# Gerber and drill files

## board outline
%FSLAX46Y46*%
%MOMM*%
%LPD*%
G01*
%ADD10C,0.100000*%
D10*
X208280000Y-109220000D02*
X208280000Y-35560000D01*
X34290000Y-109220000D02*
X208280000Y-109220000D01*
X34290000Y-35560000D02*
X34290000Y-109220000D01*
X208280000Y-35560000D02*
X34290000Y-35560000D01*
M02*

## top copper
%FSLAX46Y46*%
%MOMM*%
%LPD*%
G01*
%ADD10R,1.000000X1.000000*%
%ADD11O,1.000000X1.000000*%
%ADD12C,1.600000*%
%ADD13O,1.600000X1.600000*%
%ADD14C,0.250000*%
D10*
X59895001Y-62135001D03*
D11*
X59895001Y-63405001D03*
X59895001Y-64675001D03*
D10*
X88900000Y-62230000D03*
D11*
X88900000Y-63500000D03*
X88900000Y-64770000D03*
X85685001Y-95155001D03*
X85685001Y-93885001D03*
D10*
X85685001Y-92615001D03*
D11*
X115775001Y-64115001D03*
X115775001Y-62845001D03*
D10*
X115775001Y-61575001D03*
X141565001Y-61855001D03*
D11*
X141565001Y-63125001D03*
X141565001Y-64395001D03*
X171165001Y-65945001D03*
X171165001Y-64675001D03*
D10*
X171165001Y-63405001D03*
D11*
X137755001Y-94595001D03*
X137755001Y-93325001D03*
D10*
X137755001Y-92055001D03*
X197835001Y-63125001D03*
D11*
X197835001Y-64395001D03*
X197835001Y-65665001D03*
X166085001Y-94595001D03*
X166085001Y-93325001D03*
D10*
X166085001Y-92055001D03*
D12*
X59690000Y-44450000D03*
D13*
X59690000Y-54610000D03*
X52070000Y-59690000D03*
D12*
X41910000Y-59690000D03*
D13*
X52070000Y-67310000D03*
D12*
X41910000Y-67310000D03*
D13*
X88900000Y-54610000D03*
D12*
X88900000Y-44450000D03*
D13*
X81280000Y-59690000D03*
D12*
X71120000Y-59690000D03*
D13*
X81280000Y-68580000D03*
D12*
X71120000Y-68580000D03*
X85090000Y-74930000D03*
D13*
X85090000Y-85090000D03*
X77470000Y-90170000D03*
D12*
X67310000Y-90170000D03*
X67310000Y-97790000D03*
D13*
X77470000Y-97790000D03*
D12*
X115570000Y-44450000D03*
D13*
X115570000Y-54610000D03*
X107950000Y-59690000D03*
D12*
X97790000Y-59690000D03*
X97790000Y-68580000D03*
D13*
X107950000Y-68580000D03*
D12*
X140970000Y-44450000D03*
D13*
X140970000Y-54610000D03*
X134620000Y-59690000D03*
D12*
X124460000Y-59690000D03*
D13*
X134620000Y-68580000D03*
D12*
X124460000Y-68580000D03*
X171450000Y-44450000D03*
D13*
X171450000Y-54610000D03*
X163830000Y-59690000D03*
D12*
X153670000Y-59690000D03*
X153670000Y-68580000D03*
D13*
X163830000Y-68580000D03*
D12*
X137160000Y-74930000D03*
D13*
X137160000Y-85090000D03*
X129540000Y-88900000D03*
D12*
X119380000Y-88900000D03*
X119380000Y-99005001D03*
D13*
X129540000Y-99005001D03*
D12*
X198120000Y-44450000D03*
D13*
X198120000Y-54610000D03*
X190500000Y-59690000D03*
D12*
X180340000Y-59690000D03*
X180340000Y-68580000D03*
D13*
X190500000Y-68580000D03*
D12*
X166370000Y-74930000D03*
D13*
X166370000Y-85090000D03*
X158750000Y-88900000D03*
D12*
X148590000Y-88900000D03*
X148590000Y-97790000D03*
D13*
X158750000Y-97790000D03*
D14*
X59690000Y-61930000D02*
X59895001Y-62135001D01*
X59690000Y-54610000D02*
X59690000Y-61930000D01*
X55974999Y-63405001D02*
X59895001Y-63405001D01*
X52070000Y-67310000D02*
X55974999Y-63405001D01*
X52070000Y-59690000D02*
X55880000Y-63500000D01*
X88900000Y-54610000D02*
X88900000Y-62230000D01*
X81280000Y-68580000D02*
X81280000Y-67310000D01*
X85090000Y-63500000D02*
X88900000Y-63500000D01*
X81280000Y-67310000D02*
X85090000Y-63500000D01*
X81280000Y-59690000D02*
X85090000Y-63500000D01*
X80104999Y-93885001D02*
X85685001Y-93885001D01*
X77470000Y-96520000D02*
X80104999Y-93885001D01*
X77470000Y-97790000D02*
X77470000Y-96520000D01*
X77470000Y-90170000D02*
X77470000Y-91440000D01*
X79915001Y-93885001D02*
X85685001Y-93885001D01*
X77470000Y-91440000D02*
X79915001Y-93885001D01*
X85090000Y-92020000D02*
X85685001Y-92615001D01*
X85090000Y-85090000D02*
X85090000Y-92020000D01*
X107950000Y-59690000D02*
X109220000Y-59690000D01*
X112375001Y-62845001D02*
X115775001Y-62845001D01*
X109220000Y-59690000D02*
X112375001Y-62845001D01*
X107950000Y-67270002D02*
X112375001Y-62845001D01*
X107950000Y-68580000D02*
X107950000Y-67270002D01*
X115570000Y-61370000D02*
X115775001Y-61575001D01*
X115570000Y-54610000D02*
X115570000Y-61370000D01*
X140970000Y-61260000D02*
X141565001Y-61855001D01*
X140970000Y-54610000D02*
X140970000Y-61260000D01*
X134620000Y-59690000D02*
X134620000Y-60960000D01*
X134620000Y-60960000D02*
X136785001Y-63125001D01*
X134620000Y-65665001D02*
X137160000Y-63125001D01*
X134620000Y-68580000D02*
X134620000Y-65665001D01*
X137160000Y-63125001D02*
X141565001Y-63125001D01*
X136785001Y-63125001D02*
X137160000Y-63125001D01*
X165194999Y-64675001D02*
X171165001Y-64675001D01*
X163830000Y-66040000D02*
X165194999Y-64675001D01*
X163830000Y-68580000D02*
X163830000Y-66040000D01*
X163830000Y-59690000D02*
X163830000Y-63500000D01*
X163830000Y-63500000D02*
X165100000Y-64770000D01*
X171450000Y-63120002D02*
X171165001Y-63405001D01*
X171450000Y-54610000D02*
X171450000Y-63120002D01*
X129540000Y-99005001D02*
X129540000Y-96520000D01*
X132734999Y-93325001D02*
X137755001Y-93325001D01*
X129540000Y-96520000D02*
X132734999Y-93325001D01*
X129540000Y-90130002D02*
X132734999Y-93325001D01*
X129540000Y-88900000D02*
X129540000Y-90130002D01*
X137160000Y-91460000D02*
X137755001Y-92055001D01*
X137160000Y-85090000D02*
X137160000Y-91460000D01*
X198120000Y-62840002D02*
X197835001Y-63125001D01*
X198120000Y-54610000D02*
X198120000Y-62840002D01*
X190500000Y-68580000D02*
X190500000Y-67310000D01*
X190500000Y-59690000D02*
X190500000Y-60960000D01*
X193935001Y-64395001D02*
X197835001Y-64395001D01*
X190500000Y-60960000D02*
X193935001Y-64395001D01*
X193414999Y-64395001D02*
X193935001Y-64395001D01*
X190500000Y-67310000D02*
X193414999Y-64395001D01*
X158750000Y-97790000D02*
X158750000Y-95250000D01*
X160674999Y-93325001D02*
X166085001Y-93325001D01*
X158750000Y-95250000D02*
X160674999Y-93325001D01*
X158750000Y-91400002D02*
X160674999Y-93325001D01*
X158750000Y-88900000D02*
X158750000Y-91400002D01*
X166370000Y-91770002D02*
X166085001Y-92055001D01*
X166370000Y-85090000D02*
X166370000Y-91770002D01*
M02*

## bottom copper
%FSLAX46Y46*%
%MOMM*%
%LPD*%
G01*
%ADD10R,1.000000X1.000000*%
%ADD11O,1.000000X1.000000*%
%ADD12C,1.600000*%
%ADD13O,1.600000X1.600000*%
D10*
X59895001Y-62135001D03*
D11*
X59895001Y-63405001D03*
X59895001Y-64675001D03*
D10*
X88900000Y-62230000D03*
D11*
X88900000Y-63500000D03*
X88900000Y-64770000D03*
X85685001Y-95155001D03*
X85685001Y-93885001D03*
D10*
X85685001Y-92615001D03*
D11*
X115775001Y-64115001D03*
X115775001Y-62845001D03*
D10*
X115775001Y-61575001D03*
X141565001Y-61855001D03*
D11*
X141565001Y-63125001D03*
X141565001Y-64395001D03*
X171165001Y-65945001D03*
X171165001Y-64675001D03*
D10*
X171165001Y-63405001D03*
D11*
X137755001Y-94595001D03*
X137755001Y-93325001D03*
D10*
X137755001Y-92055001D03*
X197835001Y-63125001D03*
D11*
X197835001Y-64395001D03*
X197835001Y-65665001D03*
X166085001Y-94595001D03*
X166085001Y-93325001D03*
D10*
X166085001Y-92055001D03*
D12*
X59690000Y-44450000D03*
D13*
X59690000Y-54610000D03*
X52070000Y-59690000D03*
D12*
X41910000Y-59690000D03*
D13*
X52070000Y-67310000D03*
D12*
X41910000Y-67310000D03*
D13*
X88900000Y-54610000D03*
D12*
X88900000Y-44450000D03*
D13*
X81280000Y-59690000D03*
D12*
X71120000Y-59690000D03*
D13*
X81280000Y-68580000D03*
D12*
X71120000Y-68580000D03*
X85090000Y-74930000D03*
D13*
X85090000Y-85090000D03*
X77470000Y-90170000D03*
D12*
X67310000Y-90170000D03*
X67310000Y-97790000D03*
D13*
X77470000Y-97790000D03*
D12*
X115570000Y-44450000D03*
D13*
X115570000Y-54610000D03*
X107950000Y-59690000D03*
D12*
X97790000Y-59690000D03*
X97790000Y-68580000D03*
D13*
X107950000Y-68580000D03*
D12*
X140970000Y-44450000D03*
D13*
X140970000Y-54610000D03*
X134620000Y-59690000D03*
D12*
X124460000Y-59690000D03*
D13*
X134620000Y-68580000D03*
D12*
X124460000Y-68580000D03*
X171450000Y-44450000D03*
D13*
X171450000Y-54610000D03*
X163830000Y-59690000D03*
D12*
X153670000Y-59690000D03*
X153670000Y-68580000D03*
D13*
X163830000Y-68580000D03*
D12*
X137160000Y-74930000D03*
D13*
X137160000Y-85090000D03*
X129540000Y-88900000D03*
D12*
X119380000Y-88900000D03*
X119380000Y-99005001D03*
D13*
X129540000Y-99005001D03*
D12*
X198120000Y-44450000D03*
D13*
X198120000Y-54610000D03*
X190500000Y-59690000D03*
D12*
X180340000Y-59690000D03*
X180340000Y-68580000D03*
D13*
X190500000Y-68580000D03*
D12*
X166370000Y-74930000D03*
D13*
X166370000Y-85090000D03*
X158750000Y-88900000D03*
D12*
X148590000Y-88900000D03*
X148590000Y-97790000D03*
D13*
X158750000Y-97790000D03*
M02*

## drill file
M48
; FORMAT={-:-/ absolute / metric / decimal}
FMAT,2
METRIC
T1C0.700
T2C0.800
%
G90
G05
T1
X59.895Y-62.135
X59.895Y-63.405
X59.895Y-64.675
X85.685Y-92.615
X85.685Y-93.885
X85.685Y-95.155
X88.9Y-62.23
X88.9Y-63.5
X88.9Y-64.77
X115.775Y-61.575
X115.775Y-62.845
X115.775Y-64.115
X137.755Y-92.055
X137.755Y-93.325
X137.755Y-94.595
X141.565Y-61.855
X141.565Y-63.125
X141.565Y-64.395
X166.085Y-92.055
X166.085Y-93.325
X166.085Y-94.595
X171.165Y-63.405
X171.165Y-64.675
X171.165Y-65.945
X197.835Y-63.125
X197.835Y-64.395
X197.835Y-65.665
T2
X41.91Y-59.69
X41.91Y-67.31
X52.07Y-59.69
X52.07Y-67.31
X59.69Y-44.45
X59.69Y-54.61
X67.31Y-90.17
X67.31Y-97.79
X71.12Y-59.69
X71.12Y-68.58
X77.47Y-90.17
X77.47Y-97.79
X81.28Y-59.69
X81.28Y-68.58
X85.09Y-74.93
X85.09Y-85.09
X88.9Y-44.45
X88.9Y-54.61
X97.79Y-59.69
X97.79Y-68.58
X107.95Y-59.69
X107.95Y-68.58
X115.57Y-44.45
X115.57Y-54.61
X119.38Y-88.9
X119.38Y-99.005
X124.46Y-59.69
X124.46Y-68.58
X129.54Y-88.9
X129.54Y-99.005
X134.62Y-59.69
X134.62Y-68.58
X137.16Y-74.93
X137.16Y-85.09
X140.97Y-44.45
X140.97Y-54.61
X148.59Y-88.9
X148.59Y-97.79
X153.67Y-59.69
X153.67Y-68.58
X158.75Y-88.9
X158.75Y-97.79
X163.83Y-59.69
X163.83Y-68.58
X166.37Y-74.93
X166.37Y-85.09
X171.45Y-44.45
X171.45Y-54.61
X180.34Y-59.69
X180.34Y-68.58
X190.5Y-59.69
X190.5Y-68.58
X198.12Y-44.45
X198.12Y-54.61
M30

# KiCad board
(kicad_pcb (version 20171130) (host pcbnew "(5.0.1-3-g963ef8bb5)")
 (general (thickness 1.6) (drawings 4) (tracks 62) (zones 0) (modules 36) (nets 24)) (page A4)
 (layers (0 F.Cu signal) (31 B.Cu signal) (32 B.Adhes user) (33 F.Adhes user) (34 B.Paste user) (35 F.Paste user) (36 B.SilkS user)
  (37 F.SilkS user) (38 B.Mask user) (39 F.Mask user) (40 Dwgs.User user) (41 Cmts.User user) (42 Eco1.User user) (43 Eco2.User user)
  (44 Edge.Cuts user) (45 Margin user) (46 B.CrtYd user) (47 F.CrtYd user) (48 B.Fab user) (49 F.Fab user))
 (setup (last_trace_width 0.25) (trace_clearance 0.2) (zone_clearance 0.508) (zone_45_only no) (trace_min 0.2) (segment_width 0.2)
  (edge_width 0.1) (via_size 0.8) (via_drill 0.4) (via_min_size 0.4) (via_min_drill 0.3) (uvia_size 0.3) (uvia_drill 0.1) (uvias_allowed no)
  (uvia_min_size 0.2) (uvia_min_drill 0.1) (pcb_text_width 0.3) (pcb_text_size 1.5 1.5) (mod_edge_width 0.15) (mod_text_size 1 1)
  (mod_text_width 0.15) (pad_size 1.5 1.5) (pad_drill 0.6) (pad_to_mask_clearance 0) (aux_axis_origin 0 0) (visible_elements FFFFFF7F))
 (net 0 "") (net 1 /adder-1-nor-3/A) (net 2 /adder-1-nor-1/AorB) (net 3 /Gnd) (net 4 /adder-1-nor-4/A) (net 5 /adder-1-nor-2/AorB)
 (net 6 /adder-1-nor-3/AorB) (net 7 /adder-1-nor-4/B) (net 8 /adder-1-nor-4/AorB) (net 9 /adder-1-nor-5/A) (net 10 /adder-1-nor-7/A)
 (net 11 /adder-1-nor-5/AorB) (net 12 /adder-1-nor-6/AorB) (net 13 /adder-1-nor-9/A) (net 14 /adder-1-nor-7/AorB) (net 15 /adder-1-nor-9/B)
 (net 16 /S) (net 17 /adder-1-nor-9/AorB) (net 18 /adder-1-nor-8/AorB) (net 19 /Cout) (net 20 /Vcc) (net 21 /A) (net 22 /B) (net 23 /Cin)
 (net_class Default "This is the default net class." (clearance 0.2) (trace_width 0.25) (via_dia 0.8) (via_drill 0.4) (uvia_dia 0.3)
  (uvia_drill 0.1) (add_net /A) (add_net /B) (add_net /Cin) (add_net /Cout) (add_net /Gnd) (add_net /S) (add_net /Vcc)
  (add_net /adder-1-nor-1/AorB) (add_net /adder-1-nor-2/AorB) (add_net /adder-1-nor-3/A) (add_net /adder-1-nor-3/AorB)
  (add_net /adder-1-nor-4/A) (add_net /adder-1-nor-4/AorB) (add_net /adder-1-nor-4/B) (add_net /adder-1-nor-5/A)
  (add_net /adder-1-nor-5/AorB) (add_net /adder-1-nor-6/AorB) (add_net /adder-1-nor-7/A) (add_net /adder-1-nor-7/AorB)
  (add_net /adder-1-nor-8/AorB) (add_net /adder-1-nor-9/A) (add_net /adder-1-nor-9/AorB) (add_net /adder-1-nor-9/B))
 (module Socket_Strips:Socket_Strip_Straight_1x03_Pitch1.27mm (layer F.Cu) (at 59.895001 62.135001)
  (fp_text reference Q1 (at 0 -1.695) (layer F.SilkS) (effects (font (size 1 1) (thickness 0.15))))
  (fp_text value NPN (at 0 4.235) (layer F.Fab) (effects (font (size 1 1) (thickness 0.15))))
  (pad 1 thru_hole rect (at 0 0) (size 1 1) (drill 0.7) (layers *.Cu *.Mask) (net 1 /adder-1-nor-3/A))
  (pad 2 thru_hole oval (at 0 1.27) (size 1 1) (drill 0.7) (layers *.Cu *.Mask) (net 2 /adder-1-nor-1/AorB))
  (pad 3 thru_hole oval (at 0 2.54) (size 1 1) (drill 0.7) (layers *.Cu *.Mask) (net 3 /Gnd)))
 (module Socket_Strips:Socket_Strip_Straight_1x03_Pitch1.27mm (layer F.Cu) (at 88.9 62.23)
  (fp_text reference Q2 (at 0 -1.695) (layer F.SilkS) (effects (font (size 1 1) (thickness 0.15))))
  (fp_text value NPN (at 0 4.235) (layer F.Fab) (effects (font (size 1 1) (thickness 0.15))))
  (pad 1 thru_hole rect (at 0 0) (size 1 1) (drill 0.7) (layers *.Cu *.Mask) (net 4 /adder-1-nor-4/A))
  (pad 2 thru_hole oval (at 0 1.27) (size 1 1) (drill 0.7) (layers *.Cu *.Mask) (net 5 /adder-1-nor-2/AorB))
  (pad 3 thru_hole oval (at 0 2.54) (size 1 1) (drill 0.7) (layers *.Cu *.Mask) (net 3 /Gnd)))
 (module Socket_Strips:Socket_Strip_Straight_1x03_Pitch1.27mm (layer F.Cu) (at 85.685001 92.615001)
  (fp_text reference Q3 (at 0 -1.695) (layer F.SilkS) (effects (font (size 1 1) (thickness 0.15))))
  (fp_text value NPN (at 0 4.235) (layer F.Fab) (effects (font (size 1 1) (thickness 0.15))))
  (pad 3 thru_hole oval (at 0 2.54) (size 1 1) (drill 0.7) (layers *.Cu *.Mask) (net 3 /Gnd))
  (pad 2 thru_hole oval (at 0 1.27) (size 1 1) (drill 0.7) (layers *.Cu *.Mask) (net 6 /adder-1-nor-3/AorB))
  (pad 1 thru_hole rect (at 0 0) (size 1 1) (drill 0.7) (layers *.Cu *.Mask) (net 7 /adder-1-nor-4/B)))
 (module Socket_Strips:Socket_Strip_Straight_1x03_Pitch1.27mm (layer F.Cu) (at 115.775001 61.575001)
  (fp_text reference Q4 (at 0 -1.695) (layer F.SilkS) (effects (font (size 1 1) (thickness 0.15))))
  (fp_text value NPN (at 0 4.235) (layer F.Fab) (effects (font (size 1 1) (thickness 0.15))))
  (pad 3 thru_hole oval (at 0 2.54) (size 1 1) (drill 0.7) (layers *.Cu *.Mask) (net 3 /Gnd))
  (pad 2 thru_hole oval (at 0 1.27) (size 1 1) (drill 0.7) (layers *.Cu *.Mask) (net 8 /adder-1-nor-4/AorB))
  (pad 1 thru_hole rect (at 0 0) (size 1 1) (drill 0.7) (layers *.Cu *.Mask) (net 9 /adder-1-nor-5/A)))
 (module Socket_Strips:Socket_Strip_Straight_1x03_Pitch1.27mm (layer F.Cu) (at 141.565001 61.855001)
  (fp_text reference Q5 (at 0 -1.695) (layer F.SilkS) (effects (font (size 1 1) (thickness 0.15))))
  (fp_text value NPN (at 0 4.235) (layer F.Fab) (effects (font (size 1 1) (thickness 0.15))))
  (pad 1 thru_hole rect (at 0 0) (size 1 1) (drill 0.7) (layers *.Cu *.Mask) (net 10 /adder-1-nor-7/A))
  (pad 2 thru_hole oval (at 0 1.27) (size 1 1) (drill 0.7) (layers *.Cu *.Mask) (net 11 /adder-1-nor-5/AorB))
  (pad 3 thru_hole oval (at 0 2.54) (size 1 1) (drill 0.7) (layers *.Cu *.Mask) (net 3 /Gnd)))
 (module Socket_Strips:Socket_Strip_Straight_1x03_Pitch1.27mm (layer F.Cu) (at 171.165001 63.405001)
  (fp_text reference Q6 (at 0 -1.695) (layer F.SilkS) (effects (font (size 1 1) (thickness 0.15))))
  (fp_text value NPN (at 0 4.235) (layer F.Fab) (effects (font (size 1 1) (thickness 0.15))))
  (pad 3 thru_hole oval (at 0 2.54) (size 1 1) (drill 0.7) (layers *.Cu *.Mask) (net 3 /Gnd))
  (pad 2 thru_hole oval (at 0 1.27) (size 1 1) (drill 0.7) (layers *.Cu *.Mask) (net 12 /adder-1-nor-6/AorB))
  (pad 1 thru_hole rect (at 0 0) (size 1 1) (drill 0.7) (layers *.Cu *.Mask) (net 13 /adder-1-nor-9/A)))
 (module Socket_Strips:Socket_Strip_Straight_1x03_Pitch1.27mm (layer F.Cu) (at 137.755001 92.055001)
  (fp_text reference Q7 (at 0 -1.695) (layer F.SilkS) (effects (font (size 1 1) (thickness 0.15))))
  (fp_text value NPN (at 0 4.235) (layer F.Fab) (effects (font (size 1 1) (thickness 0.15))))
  (pad 3 thru_hole oval (at 0 2.54) (size 1 1) (drill 0.7) (layers *.Cu *.Mask) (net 3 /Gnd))
  (pad 2 thru_hole oval (at 0 1.27) (size 1 1) (drill 0.7) (layers *.Cu *.Mask) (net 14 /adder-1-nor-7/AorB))
  (pad 1 thru_hole rect (at 0 0) (size 1 1) (drill 0.7) (layers *.Cu *.Mask) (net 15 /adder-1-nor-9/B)))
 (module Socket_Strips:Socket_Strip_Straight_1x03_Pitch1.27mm (layer F.Cu) (at 197.835001 63.125001)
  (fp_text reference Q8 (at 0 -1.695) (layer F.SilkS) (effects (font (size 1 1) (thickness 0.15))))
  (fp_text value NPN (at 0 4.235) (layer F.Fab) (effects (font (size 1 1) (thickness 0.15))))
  (pad 1 thru_hole rect (at 0 0) (size 1 1) (drill 0.7) (layers *.Cu *.Mask) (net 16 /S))
  (pad 2 thru_hole oval (at 0 1.27) (size 1 1) (drill 0.7) (layers *.Cu *.Mask) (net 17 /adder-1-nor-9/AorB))
  (pad 3 thru_hole oval (at 0 2.54) (size 1 1) (drill 0.7) (layers *.Cu *.Mask) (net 3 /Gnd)))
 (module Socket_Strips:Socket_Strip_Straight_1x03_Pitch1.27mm (layer F.Cu) (at 166.085001 92.055001)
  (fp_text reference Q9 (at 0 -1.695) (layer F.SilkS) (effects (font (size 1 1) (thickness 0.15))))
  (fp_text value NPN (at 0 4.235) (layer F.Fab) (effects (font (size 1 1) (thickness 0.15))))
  (pad 3 thru_hole oval (at 0 2.54) (size 1 1) (drill 0.7) (layers *.Cu *.Mask) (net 3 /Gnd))
  (pad 2 thru_hole oval (at 0 1.27) (size 1 1) (drill 0.7) (layers *.Cu *.Mask) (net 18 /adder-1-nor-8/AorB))
  (pad 1 thru_hole rect (at 0 0) (size 1 1) (drill 0.7) (layers *.Cu *.Mask) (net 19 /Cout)))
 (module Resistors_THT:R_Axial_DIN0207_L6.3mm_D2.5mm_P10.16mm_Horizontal (layer F.Cu) (at 59.69 44.45 270)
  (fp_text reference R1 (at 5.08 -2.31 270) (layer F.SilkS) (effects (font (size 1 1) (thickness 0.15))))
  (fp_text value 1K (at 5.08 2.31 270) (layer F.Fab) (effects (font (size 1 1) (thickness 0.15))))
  (pad 1 thru_hole circle (at 0 0 270) (size 1.6 1.6) (drill 0.8) (layers *.Cu *.Mask) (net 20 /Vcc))
  (pad 2 thru_hole oval (at 10.16 0 270) (size 1.6 1.6) (drill 0.8) (layers *.Cu *.Mask) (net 1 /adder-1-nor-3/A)))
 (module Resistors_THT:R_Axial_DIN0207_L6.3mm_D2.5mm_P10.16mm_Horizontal (layer F.Cu) (at 41.91 59.69)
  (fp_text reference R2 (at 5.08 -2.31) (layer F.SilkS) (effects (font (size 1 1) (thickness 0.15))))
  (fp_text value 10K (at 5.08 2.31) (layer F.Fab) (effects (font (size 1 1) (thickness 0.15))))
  (pad 2 thru_hole oval (at 10.16 0) (size 1.6 1.6) (drill 0.8) (layers *.Cu *.Mask) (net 2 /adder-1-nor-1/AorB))
  (pad 1 thru_hole circle (at 0 0) (size 1.6 1.6) (drill 0.8) (layers *.Cu *.Mask) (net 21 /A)))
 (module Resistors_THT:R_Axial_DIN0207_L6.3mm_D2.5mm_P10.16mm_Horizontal (layer F.Cu) (at 41.91 67.31)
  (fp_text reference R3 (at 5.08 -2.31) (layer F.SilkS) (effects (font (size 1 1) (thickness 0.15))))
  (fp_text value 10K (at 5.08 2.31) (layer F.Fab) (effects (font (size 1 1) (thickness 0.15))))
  (pad 2 thru_hole oval (at 10.16 0) (size 1.6 1.6) (drill 0.8) (layers *.Cu *.Mask) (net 2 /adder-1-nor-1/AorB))
  (pad 1 thru_hole circle (at 0 0) (size 1.6 1.6) (drill 0.8) (layers *.Cu *.Mask) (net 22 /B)))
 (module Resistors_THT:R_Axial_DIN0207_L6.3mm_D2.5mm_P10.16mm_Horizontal (layer F.Cu) (at 88.9 44.45 270)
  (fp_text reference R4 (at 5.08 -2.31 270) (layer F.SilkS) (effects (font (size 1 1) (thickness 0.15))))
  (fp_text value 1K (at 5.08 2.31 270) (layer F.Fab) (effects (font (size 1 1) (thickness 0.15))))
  (pad 2 thru_hole oval (at 10.16 0 270) (size 1.6 1.6) (drill 0.8) (layers *.Cu *.Mask) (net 4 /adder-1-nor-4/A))
  (pad 1 thru_hole circle (at 0 0 270) (size 1.6 1.6) (drill 0.8) (layers *.Cu *.Mask) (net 20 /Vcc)))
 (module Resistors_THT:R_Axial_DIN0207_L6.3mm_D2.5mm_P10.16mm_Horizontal (layer F.Cu) (at 71.12 59.69)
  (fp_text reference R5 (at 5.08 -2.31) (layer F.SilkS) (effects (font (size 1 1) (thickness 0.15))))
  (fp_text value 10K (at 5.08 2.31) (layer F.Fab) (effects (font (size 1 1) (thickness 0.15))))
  (pad 2 thru_hole oval (at 10.16 0) (size 1.6 1.6) (drill 0.8) (layers *.Cu *.Mask) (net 5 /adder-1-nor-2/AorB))
  (pad 1 thru_hole circle (at 0 0) (size 1.6 1.6) (drill 0.8) (layers *.Cu *.Mask) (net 21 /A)))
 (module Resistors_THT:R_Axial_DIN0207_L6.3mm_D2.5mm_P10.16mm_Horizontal (layer F.Cu) (at 71.12 68.58)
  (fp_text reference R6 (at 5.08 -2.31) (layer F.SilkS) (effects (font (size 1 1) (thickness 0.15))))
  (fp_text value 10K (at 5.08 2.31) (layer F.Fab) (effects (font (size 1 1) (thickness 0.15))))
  (pad 2 thru_hole oval (at 10.16 0) (size 1.6 1.6) (drill 0.8) (layers *.Cu *.Mask) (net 5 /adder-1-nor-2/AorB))
  (pad 1 thru_hole circle (at 0 0) (size 1.6 1.6) (drill 0.8) (layers *.Cu *.Mask) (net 1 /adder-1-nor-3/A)))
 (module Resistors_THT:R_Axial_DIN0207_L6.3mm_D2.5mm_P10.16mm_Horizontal (layer F.Cu) (at 85.09 74.93 270)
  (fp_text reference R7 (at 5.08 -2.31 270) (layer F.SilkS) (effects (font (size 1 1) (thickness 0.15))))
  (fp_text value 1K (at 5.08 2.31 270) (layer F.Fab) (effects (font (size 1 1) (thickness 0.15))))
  (pad 1 thru_hole circle (at 0 0 270) (size 1.6 1.6) (drill 0.8) (layers *.Cu *.Mask) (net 20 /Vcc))
  (pad 2 thru_hole oval (at 10.16 0 270) (size 1.6 1.6) (drill 0.8) (layers *.Cu *.Mask) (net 7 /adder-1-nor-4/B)))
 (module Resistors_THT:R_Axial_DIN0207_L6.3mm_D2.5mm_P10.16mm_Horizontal (layer F.Cu) (at 67.31 90.17)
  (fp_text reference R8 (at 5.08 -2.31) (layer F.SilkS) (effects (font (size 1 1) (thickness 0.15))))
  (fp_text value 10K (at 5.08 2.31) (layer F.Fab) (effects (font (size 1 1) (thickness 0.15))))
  (pad 2 thru_hole oval (at 10.16 0) (size 1.6 1.6) (drill 0.8) (layers *.Cu *.Mask) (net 6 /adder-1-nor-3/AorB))
  (pad 1 thru_hole circle (at 0 0) (size 1.6 1.6) (drill 0.8) (layers *.Cu *.Mask) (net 1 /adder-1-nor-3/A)))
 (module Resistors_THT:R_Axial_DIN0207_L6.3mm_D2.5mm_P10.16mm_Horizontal (layer F.Cu) (at 67.31 97.79)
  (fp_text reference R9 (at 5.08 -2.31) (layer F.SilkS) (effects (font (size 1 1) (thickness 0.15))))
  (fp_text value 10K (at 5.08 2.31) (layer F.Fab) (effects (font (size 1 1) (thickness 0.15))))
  (pad 1 thru_hole circle (at 0 0) (size 1.6 1.6) (drill 0.8) (layers *.Cu *.Mask) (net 22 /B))
  (pad 2 thru_hole oval (at 10.16 0) (size 1.6 1.6) (drill 0.8) (layers *.Cu *.Mask) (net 6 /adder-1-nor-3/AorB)))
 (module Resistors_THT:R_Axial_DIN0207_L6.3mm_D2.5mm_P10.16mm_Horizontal (layer F.Cu) (at 115.57 44.45 270)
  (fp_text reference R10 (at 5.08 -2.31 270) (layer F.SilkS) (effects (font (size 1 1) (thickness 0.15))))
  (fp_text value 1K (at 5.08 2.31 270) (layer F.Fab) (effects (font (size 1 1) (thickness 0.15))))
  (pad 1 thru_hole circle (at 0 0 270) (size 1.6 1.6) (drill 0.8) (layers *.Cu *.Mask) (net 20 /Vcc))
  (pad 2 thru_hole oval (at 10.16 0 270) (size 1.6 1.6) (drill 0.8) (layers *.Cu *.Mask) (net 9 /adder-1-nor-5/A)))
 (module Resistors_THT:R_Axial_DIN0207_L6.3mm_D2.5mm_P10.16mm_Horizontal (layer F.Cu) (at 97.79 59.69)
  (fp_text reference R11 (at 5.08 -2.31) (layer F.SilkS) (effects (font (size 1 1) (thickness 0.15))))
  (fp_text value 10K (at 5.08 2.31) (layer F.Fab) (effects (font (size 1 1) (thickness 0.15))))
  (pad 2 thru_hole oval (at 10.16 0) (size 1.6 1.6) (drill 0.8) (layers *.Cu *.Mask) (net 8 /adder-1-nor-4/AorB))
  (pad 1 thru_hole circle (at 0 0) (size 1.6 1.6) (drill 0.8) (layers *.Cu *.Mask) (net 4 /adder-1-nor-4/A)))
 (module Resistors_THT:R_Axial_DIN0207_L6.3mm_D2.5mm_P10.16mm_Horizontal (layer F.Cu) (at 97.79 68.58)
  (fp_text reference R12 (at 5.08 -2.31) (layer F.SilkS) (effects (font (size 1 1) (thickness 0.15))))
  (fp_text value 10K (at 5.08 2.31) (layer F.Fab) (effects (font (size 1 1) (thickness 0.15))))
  (pad 1 thru_hole circle (at 0 0) (size 1.6 1.6) (drill 0.8) (layers *.Cu *.Mask) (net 7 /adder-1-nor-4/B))
  (pad 2 thru_hole oval (at 10.16 0) (size 1.6 1.6) (drill 0.8) (layers *.Cu *.Mask) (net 8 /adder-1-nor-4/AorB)))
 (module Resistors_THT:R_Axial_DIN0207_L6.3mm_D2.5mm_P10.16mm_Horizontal (layer F.Cu) (at 140.97 44.45 270)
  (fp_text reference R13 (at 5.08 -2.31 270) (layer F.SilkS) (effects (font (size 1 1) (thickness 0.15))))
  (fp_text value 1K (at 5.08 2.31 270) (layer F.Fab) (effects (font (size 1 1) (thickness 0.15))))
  (pad 1 thru_hole circle (at 0 0 270) (size 1.6 1.6) (drill 0.8) (layers *.Cu *.Mask) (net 20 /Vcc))
  (pad 2 thru_hole oval (at 10.16 0 270) (size 1.6 1.6) (drill 0.8) (layers *.Cu *.Mask) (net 10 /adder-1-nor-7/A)))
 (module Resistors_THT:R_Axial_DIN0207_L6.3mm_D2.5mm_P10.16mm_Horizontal (layer F.Cu) (at 124.46 59.69)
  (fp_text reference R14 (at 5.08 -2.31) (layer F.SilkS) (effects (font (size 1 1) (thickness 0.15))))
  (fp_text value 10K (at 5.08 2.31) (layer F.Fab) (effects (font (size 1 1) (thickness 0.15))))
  (pad 2 thru_hole oval (at 10.16 0) (size 1.6 1.6) (drill 0.8) (layers *.Cu *.Mask) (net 11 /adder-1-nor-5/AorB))
  (pad 1 thru_hole circle (at 0 0) (size 1.6 1.6) (drill 0.8) (layers *.Cu *.Mask) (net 9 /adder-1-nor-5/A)))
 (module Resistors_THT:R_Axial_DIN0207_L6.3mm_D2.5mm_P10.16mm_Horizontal (layer F.Cu) (at 124.46 68.58)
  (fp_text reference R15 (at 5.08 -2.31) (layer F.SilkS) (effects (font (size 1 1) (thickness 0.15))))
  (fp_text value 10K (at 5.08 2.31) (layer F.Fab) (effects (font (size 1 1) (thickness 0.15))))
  (pad 2 thru_hole oval (at 10.16 0) (size 1.6 1.6) (drill 0.8) (layers *.Cu *.Mask) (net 11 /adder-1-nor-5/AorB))
  (pad 1 thru_hole circle (at 0 0) (size 1.6 1.6) (drill 0.8) (layers *.Cu *.Mask) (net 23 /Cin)))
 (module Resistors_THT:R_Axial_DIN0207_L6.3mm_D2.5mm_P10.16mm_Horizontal (layer F.Cu) (at 171.45 44.45 270)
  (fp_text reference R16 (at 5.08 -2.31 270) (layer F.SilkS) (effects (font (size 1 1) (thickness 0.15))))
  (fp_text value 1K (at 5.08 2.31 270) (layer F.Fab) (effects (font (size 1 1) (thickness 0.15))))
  (pad 1 thru_hole circle (at 0 0 270) (size 1.6 1.6) (drill 0.8) (layers *.Cu *.Mask) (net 20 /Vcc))
  (pad 2 thru_hole oval (at 10.16 0 270) (size 1.6 1.6) (drill 0.8) (layers *.Cu *.Mask) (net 13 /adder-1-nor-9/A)))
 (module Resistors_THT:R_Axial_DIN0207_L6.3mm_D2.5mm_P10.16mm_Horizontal (layer F.Cu) (at 153.67 59.69)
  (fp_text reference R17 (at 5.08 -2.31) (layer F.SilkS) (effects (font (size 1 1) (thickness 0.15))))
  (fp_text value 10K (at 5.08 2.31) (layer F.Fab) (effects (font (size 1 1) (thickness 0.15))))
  (pad 2 thru_hole oval (at 10.16 0) (size 1.6 1.6) (drill 0.8) (layers *.Cu *.Mask) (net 12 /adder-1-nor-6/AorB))
  (pad 1 thru_hole circle (at 0 0) (size 1.6 1.6) (drill 0.8) (layers *.Cu *.Mask) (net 9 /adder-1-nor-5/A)))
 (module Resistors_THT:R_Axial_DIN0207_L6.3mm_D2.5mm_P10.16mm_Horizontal (layer F.Cu) (at 153.67 68.58)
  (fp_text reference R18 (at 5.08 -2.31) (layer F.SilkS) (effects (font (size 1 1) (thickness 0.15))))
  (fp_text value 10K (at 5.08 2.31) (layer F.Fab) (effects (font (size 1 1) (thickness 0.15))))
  (pad 1 thru_hole circle (at 0 0) (size 1.6 1.6) (drill 0.8) (layers *.Cu *.Mask) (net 10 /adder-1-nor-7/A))
  (pad 2 thru_hole oval (at 10.16 0) (size 1.6 1.6) (drill 0.8) (layers *.Cu *.Mask) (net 12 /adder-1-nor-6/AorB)))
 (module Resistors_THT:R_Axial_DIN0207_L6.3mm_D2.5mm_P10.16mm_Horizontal (layer F.Cu) (at 137.16 74.93 270)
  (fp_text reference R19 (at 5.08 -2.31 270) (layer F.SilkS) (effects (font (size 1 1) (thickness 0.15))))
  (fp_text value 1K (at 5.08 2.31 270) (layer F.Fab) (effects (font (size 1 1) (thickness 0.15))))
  (pad 1 thru_hole circle (at 0 0 270) (size 1.6 1.6) (drill 0.8) (layers *.Cu *.Mask) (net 20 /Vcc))
  (pad 2 thru_hole oval (at 10.16 0 270) (size 1.6 1.6) (drill 0.8) (layers *.Cu *.Mask) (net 15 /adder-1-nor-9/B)))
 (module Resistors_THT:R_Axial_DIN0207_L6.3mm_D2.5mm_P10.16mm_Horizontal (layer F.Cu) (at 119.38 88.9)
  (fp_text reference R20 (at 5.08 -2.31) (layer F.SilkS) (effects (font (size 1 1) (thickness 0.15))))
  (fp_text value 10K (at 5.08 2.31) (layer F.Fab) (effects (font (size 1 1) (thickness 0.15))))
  (pad 2 thru_hole oval (at 10.16 0) (size 1.6 1.6) (drill 0.8) (layers *.Cu *.Mask) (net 14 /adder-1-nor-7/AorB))
  (pad 1 thru_hole circle (at 0 0) (size 1.6 1.6) (drill 0.8) (layers *.Cu *.Mask) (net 10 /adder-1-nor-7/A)))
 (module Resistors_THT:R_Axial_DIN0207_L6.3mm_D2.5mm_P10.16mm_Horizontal (layer F.Cu) (at 119.38 99.005001)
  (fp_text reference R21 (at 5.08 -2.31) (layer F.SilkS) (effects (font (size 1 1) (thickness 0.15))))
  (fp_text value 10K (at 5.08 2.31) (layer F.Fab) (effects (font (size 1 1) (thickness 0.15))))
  (pad 1 thru_hole circle (at 0 0) (size 1.6 1.6) (drill 0.8) (layers *.Cu *.Mask) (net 23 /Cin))
  (pad 2 thru_hole oval (at 10.16 0) (size 1.6 1.6) (drill 0.8) (layers *.Cu *.Mask) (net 14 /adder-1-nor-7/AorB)))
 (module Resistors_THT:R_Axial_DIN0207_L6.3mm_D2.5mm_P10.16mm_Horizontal (layer F.Cu) (at 198.12 44.45 270)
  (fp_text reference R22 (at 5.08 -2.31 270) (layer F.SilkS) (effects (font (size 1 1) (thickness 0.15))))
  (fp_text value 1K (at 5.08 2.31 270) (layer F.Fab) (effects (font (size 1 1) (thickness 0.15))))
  (pad 1 thru_hole circle (at 0 0 270) (size 1.6 1.6) (drill 0.8) (layers *.Cu *.Mask) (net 20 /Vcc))
  (pad 2 thru_hole oval (at 10.16 0 270) (size 1.6 1.6) (drill 0.8) (layers *.Cu *.Mask) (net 16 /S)))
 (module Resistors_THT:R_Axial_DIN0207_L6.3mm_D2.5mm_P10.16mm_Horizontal (layer F.Cu) (at 180.34 59.69)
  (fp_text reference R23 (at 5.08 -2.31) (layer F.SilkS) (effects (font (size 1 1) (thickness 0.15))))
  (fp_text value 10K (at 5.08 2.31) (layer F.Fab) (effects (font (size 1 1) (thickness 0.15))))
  (pad 2 thru_hole oval (at 10.16 0) (size 1.6 1.6) (drill 0.8) (layers *.Cu *.Mask) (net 17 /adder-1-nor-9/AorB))
  (pad 1 thru_hole circle (at 0 0) (size 1.6 1.6) (drill 0.8) (layers *.Cu *.Mask) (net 13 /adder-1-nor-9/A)))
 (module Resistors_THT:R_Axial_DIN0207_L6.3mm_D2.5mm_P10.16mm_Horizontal (layer F.Cu) (at 180.34 68.58)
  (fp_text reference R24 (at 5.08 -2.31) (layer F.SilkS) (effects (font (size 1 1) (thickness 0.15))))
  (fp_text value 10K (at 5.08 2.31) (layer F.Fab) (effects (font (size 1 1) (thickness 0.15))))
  (pad 1 thru_hole circle (at 0 0) (size 1.6 1.6) (drill 0.8) (layers *.Cu *.Mask) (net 15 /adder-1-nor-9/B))
  (pad 2 thru_hole oval (at 10.16 0) (size 1.6 1.6) (drill 0.8) (layers *.Cu *.Mask) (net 17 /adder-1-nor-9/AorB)))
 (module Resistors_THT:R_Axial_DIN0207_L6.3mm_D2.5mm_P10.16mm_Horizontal (layer F.Cu) (at 166.37 74.93 270)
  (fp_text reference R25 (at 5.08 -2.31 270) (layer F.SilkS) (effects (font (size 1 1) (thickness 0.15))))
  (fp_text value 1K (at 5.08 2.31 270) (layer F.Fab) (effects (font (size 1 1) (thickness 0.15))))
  (pad 1 thru_hole circle (at 0 0 270) (size 1.6 1.6) (drill 0.8) (layers *.Cu *.Mask) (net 20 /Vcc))
  (pad 2 thru_hole oval (at 10.16 0 270) (size 1.6 1.6) (drill 0.8) (layers *.Cu *.Mask) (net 19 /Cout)))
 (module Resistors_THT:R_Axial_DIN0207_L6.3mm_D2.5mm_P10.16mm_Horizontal (layer F.Cu) (at 148.59 88.9)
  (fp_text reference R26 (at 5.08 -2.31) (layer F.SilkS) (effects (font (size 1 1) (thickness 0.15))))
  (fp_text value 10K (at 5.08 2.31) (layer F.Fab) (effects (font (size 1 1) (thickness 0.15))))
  (pad 2 thru_hole oval (at 10.16 0) (size 1.6 1.6) (drill 0.8) (layers *.Cu *.Mask) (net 18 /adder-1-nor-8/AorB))
  (pad 1 thru_hole circle (at 0 0) (size 1.6 1.6) (drill 0.8) (layers *.Cu *.Mask) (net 10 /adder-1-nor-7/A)))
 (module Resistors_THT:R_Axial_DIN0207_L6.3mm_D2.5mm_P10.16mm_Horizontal (layer F.Cu) (at 148.59 97.79)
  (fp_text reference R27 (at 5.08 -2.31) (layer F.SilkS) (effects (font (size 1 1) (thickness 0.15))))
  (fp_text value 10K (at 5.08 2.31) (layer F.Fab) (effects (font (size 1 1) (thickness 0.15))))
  (pad 1 thru_hole circle (at 0 0) (size 1.6 1.6) (drill 0.8) (layers *.Cu *.Mask) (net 1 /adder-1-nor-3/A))
  (pad 2 thru_hole oval (at 10.16 0) (size 1.6 1.6) (drill 0.8) (layers *.Cu *.Mask) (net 18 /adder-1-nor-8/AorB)))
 (gr_line (start 208.28 109.22) (end 208.28 35.56) (layer Edge.Cuts) (width 0.1))
 (gr_line (start 34.29 109.22) (end 208.28 109.22) (layer Edge.Cuts) (width 0.1))
 (gr_line (start 34.29 35.56) (end 34.29 109.22) (layer Edge.Cuts) (width 0.1))
 (gr_line (start 208.28 35.56) (end 34.29 35.56) (layer Edge.Cuts) (width 0.1))
 (segment (start 59.69 61.93) (end 59.895001 62.135001) (width 0.25) (layer F.Cu) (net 1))
 (segment (start 59.69 54.61) (end 59.69 61.93) (width 0.25) (layer F.Cu) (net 1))
 (segment (start 55.974999 63.405001) (end 59.895001 63.405001) (width 0.25) (layer F.Cu) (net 2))
 (segment (start 52.07 67.31) (end 55.974999 63.405001) (width 0.25) (layer F.Cu) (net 2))
 (segment (start 52.07 59.69) (end 55.88 63.5) (width 0.25) (layer F.Cu) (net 2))
 (segment (start 88.9 54.61) (end 88.9 62.23) (width 0.25) (layer F.Cu) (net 4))
 (segment (start 81.28 68.58) (end 81.28 67.31) (width 0.25) (layer F.Cu) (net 5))
 (segment (start 85.09 63.5) (end 88.9 63.5) (width 0.25) (layer F.Cu) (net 5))
 (segment (start 81.28 67.31) (end 85.09 63.5) (width 0.25) (layer F.Cu) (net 5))
 (segment (start 81.28 59.69) (end 85.09 63.5) (width 0.25) (layer F.Cu) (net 5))
 (segment (start 80.104999 93.885001) (end 85.685001 93.885001) (width 0.25) (layer F.Cu) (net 6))
 (segment (start 77.47 96.52) (end 80.104999 93.885001) (width 0.25) (layer F.Cu) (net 6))
 (segment (start 77.47 97.79) (end 77.47 96.52) (width 0.25) (layer F.Cu) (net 6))
 (segment (start 77.47 90.17) (end 77.47 91.44) (width 0.25) (layer F.Cu) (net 6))
 (segment (start 79.915001 93.885001) (end 85.685001 93.885001) (width 0.25) (layer F.Cu) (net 6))
 (segment (start 77.47 91.44) (end 79.915001 93.885001) (width 0.25) (layer F.Cu) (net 6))
 (segment (start 85.09 92.02) (end 85.685001 92.615001) (width 0.25) (layer F.Cu) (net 7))
 (segment (start 85.09 85.09) (end 85.09 92.02) (width 0.25) (layer F.Cu) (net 7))
 (segment (start 107.95 59.69) (end 109.22 59.69) (width 0.25) (layer F.Cu) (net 8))
 (segment (start 112.375001 62.845001) (end 115.775001 62.845001) (width 0.25) (layer F.Cu) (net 8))
 (segment (start 109.22 59.69) (end 112.375001 62.845001) (width 0.25) (layer F.Cu) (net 8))
 (segment (start 107.95 67.270002) (end 112.375001 62.845001) (width 0.25) (layer F.Cu) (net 8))
 (segment (start 107.95 68.58) (end 107.95 67.270002) (width 0.25) (layer F.Cu) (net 8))
 (segment (start 115.57 61.37) (end 115.775001 61.575001) (width 0.25) (layer F.Cu) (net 9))
 (segment (start 115.57 54.61) (end 115.57 61.37) (width 0.25) (layer F.Cu) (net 9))
 (segment (start 140.97 61.26) (end 141.565001 61.855001) (width 0.25) (layer F.Cu) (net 10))
 (segment (start 140.97 54.61) (end 140.97 61.26) (width 0.25) (layer F.Cu) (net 10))
 (segment (start 134.62 59.69) (end 134.62 60.96) (width 0.25) (layer F.Cu) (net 11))
 (segment (start 134.62 60.96) (end 136.785001 63.125001) (width 0.25) (layer F.Cu) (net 11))
 (segment (start 134.62 65.665001) (end 137.16 63.125001) (width 0.25) (layer F.Cu) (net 11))
 (segment (start 134.62 68.58) (end 134.62 65.665001) (width 0.25) (layer F.Cu) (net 11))
 (segment (start 137.16 63.125001) (end 141.565001 63.125001) (width 0.25) (layer F.Cu) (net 11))
 (segment (start 136.785001 63.125001) (end 137.16 63.125001) (width 0.25) (layer F.Cu) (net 11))
 (segment (start 165.194999 64.675001) (end 171.165001 64.675001) (width 0.25) (layer F.Cu) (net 12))
 (segment (start 163.83 66.04) (end 165.194999 64.675001) (width 0.25) (layer F.Cu) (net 12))
 (segment (start 163.83 68.58) (end 163.83 66.04) (width 0.25) (layer F.Cu) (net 12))
 (segment (start 163.83 59.69) (end 163.83 63.5) (width 0.25) (layer F.Cu) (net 12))
 (segment (start 163.83 63.5) (end 165.1 64.77) (width 0.25) (layer F.Cu) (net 12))
 (segment (start 171.45 63.120002) (end 171.165001 63.405001) (width 0.25) (layer F.Cu) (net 13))
 (segment (start 171.45 54.61) (end 171.45 63.120002) (width 0.25) (layer F.Cu) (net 13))
 (segment (start 129.54 99.005001) (end 129.54 96.52) (width 0.25) (layer F.Cu) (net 14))
 (segment (start 132.734999 93.325001) (end 137.755001 93.325001) (width 0.25) (layer F.Cu) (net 14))
 (segment (start 129.54 96.52) (end 132.734999 93.325001) (width 0.25) (layer F.Cu) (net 14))
 (segment (start 129.54 90.130002) (end 132.734999 93.325001) (width 0.25) (layer F.Cu) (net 14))
 (segment (start 129.54 88.9) (end 129.54 90.130002) (width 0.25) (layer F.Cu) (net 14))
 (segment (start 137.16 91.46) (end 137.755001 92.055001) (width 0.25) (layer F.Cu) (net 15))
 (segment (start 137.16 85.09) (end 137.16 91.46) (width 0.25) (layer F.Cu) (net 15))
 (segment (start 198.12 62.840002) (end 197.835001 63.125001) (width 0.25) (layer F.Cu) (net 16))
 (segment (start 198.12 54.61) (end 198.12 62.840002) (width 0.25) (layer F.Cu) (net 16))
 (segment (start 190.5 68.58) (end 190.5 67.31) (width 0.25) (layer F.Cu) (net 17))
 (segment (start 190.5 59.69) (end 190.5 60.96) (width 0.25) (layer F.Cu) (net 17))
 (segment (start 193.935001 64.395001) (end 197.835001 64.395001) (width 0.25) (layer F.Cu) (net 17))
 (segment (start 190.5 60.96) (end 193.935001 64.395001) (width 0.25) (layer F.Cu) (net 17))
 (segment (start 193.414999 64.395001) (end 193.935001 64.395001) (width 0.25) (layer F.Cu) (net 17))
 (segment (start 190.5 67.31) (end 193.414999 64.395001) (width 0.25) (layer F.Cu) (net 17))
 (segment (start 158.75 97.79) (end 158.75 95.25) (width 0.25) (layer F.Cu) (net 18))
 (segment (start 160.674999 93.325001) (end 166.085001 93.325001) (width 0.25) (layer F.Cu) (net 18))
 (segment (start 158.75 95.25) (end 160.674999 93.325001) (width 0.25) (layer F.Cu) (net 18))
 (segment (start 158.75 91.400002) (end 160.674999 93.325001) (width 0.25) (layer F.Cu) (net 18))
 (segment (start 158.75 88.9) (end 158.75 91.400002) (width 0.25) (layer F.Cu) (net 18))
 (segment (start 166.37 91.770002) (end 166.085001 92.055001) (width 0.25) (layer F.Cu) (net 19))
 (segment (start 166.37 85.09) (end 166.37 91.770002) (width 0.25) (layer F.Cu) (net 19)))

